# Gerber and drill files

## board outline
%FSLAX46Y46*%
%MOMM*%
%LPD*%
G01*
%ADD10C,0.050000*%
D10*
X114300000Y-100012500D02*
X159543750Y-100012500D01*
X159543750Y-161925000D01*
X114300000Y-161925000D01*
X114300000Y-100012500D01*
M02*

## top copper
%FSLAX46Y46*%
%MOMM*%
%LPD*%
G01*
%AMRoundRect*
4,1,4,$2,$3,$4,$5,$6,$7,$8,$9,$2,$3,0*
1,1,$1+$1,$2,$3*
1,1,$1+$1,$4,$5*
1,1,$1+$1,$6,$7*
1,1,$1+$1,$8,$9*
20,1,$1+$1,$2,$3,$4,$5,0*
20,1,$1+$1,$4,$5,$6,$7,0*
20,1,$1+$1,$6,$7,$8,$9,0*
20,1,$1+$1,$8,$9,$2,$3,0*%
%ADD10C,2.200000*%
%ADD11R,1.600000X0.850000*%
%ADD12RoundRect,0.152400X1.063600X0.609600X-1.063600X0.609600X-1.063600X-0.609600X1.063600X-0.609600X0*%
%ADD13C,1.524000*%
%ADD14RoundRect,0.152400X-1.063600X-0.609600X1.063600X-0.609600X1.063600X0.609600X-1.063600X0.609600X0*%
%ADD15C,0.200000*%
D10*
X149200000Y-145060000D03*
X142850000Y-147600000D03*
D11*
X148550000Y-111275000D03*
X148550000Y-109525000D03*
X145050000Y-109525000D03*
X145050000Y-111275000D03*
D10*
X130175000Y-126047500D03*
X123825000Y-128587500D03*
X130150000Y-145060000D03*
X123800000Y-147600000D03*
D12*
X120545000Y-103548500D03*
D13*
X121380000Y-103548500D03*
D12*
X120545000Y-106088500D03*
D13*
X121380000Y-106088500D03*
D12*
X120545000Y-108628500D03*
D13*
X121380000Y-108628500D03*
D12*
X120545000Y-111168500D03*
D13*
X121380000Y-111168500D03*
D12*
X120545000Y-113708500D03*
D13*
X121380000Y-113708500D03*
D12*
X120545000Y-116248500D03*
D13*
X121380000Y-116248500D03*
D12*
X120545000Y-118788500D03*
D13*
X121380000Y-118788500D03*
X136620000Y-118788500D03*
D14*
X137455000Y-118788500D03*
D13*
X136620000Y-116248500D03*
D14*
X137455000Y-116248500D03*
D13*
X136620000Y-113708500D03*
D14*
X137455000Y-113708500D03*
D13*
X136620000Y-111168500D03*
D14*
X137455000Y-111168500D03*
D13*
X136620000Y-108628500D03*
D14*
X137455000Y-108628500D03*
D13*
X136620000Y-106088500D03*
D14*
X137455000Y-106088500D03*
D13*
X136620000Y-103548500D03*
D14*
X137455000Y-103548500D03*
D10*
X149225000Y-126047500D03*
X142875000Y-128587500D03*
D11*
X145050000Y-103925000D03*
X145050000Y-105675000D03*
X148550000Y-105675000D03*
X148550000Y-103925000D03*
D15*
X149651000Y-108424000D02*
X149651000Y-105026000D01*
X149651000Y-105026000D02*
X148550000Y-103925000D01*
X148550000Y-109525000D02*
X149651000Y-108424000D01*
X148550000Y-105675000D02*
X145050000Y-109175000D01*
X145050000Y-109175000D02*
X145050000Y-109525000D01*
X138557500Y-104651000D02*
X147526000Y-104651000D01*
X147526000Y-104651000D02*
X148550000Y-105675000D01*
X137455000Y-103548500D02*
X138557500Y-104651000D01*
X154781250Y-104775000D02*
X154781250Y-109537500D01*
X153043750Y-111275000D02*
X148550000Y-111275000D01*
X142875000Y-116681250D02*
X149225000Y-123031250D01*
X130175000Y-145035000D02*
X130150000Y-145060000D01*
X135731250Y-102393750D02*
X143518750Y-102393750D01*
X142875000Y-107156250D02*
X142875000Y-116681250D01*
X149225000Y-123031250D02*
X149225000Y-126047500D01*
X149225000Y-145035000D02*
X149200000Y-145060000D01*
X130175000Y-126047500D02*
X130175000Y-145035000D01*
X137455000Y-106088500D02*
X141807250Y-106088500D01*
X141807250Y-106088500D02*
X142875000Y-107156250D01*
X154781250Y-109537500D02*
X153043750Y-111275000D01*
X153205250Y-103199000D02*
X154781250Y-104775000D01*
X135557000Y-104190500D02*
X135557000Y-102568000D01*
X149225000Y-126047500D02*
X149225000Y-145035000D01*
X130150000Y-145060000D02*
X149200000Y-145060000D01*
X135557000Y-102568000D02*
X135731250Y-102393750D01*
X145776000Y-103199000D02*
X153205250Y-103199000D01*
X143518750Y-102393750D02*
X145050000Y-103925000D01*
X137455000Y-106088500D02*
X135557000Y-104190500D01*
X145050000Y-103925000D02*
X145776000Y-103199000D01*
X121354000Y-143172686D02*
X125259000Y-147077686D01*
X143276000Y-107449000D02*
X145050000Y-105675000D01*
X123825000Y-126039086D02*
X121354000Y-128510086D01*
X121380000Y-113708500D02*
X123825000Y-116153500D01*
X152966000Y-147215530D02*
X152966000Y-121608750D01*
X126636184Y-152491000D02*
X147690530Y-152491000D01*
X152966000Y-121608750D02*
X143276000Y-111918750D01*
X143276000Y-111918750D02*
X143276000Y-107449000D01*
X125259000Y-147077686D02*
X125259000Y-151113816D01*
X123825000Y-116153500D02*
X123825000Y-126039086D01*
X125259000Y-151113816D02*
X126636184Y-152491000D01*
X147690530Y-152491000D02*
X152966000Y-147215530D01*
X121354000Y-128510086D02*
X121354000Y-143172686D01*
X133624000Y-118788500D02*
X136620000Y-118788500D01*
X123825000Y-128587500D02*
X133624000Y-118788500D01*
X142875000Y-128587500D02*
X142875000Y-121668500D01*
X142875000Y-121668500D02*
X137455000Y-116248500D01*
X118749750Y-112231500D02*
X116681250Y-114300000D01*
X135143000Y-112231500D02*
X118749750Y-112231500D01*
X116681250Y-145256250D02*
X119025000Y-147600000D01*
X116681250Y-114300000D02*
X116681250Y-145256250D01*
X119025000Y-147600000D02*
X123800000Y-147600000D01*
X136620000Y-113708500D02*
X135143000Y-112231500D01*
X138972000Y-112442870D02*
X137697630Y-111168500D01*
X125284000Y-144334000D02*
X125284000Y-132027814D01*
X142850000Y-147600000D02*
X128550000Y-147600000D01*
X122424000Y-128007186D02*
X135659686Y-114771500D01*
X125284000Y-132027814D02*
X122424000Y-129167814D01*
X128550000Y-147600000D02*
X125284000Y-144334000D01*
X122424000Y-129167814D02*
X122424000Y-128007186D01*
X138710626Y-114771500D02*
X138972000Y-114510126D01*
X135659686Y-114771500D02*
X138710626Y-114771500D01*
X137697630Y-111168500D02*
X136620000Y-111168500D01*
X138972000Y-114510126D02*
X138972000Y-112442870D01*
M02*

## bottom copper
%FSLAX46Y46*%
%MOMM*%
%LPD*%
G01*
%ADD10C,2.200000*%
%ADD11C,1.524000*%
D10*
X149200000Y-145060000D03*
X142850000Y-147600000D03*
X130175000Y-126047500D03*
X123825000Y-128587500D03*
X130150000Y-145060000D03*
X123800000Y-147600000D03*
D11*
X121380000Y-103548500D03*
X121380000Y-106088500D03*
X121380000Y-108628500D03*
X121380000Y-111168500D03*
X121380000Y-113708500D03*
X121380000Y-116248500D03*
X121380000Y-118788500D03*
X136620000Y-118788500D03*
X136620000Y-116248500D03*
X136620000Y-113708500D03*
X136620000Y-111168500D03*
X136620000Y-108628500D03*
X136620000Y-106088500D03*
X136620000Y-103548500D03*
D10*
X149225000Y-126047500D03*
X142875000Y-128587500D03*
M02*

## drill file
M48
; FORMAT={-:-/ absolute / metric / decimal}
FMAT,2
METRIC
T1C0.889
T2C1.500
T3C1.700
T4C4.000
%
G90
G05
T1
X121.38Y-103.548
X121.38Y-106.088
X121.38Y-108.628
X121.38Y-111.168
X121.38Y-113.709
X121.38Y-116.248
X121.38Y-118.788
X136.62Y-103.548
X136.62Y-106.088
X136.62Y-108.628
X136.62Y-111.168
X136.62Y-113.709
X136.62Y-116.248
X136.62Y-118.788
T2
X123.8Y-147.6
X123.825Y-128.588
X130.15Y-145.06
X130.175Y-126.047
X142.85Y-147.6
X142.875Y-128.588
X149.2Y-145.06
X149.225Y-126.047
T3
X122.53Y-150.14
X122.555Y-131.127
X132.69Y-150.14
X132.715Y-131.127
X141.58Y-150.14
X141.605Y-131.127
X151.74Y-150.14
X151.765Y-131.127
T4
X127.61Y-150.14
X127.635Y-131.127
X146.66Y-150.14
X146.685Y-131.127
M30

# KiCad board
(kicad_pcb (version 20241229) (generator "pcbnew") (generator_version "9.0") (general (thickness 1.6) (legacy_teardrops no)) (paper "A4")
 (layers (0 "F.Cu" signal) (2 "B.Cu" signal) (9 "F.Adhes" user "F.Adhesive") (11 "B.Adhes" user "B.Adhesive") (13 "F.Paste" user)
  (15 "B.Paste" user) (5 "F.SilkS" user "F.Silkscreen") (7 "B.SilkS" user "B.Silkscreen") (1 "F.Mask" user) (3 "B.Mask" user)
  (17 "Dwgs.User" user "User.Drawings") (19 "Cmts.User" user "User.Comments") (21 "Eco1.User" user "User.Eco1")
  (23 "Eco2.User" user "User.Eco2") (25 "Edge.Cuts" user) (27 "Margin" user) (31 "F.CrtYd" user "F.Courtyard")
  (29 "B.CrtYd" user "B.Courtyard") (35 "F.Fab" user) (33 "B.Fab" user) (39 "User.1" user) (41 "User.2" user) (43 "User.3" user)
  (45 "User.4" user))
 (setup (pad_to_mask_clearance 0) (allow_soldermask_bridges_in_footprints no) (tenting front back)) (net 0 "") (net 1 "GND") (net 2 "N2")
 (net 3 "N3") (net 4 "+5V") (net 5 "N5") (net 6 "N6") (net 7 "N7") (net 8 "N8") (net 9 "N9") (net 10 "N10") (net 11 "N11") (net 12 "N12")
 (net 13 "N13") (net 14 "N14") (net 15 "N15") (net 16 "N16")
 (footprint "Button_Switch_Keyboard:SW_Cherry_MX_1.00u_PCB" (layer "F.Cu") (at 149.2 145.06)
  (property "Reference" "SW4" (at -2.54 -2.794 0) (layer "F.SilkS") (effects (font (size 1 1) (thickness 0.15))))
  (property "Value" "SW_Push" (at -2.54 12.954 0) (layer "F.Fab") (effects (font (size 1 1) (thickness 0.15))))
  (pad "" np_thru_hole circle (at -7.62 5.08) (size 1.7 1.7) (drill 1.7) (layers "*.Cu" "*.Mask"))
  (pad "" np_thru_hole circle (at -2.54 5.08) (size 4 4) (drill 4) (layers "*.Cu" "*.Mask"))
  (pad "" np_thru_hole circle (at 2.54 5.08) (size 1.7 1.7) (drill 1.7) (layers "*.Cu" "*.Mask"))
  (pad "1" thru_hole circle (at 0 0) (size 2.2 2.2) (drill 1.5) (layers "*.Cu" "*.Mask") (remove_unused_layers no) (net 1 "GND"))
  (pad "2" thru_hole circle (at -6.35 2.54) (size 2.2 2.2) (drill 1.5) (layers "*.Cu" "*.Mask") (remove_unused_layers no) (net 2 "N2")))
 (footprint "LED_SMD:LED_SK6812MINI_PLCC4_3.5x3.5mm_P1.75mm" (layer "F.Cu") (at 146.8 110.4 180)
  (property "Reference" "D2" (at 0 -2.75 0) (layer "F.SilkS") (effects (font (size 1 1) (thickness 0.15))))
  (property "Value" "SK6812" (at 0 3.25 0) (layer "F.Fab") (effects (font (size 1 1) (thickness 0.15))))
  (pad "1" smd rect (at -1.75 -0.875 180) (size 1.6 0.85) (layers "F.Cu" "F.Mask" "F.Paste") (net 1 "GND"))
  (pad "2" smd rect (at -1.75 0.875 180) (size 1.6 0.85) (layers "F.Cu" "F.Mask" "F.Paste") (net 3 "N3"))
  (pad "3" smd rect (at 1.75 0.875 180) (size 1.6 0.85) (layers "F.Cu" "F.Mask" "F.Paste") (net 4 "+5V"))
  (pad "4" smd rect (at 1.75 -0.875 180) (size 1.6 0.85) (layers "F.Cu" "F.Mask" "F.Paste") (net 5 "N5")))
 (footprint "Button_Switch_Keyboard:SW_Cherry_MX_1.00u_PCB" (layer "F.Cu") (at 130.175 126.0475)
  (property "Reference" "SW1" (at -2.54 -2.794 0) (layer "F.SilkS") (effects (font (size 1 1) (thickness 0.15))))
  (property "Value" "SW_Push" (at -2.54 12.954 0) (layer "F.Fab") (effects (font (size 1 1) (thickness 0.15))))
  (pad "" np_thru_hole circle (at -7.62 5.08) (size 1.7 1.7) (drill 1.7) (layers "*.Cu" "*.Mask"))
  (pad "" np_thru_hole circle (at -2.54 5.08) (size 4 4) (drill 4) (layers "*.Cu" "*.Mask"))
  (pad "" np_thru_hole circle (at 2.54 5.08) (size 1.7 1.7) (drill 1.7) (layers "*.Cu" "*.Mask"))
  (pad "1" thru_hole circle (at 0 0) (size 2.2 2.2) (drill 1.5) (layers "*.Cu" "*.Mask") (remove_unused_layers no) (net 1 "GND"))
  (pad "2" thru_hole circle (at -6.35 2.54) (size 2.2 2.2) (drill 1.5) (layers "*.Cu" "*.Mask") (remove_unused_layers no) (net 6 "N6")))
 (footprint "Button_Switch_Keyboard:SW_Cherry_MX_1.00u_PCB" (layer "F.Cu") (at 130.15 145.06)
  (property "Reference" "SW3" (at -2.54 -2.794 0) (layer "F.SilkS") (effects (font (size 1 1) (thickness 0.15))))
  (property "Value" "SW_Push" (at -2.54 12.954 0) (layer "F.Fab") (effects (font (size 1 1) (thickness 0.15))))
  (pad "" np_thru_hole circle (at -7.62 5.08) (size 1.7 1.7) (drill 1.7) (layers "*.Cu" "*.Mask"))
  (pad "" np_thru_hole circle (at -2.54 5.08) (size 4 4) (drill 4) (layers "*.Cu" "*.Mask"))
  (pad "" np_thru_hole circle (at 2.54 5.08) (size 1.7 1.7) (drill 1.7) (layers "*.Cu" "*.Mask"))
  (pad "1" thru_hole circle (at 0 0) (size 2.2 2.2) (drill 1.5) (layers "*.Cu" "*.Mask") (remove_unused_layers no) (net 1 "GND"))
  (pad "2" thru_hole circle (at -6.35 2.54) (size 2.2 2.2) (drill 1.5) (layers "*.Cu" "*.Mask") (remove_unused_layers no) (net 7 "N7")))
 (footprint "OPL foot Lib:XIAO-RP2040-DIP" (layer "F.Cu") (at 129 111.1685)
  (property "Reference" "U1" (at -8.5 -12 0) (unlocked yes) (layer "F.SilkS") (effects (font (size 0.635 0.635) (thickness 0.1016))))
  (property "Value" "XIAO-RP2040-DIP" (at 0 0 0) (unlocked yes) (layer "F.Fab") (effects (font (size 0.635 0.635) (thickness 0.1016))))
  (pad "1" smd roundrect (at -8.455 -7.62 180) (size 2.432 1.524) (layers "F.Cu" "F.Mask") (roundrect_rratio 0.1) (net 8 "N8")
   (thermal_bridge_angle 45))
  (pad "1" thru_hole circle (at -7.62 -7.62 180) (size 1.524 1.524) (drill 0.889) (layers "*.Cu" "*.Mask") (remove_unused_layers no)
   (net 8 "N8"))
  (pad "2" smd roundrect (at -8.455 -5.08 180) (size 2.432 1.524) (layers "F.Cu" "F.Mask") (roundrect_rratio 0.1) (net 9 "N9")
   (thermal_bridge_angle 45))
  (pad "2" thru_hole circle (at -7.62 -5.08 180) (size 1.524 1.524) (drill 0.889) (layers "*.Cu" "*.Mask") (remove_unused_layers no)
   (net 9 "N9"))
  (pad "3" smd roundrect (at -8.455 -2.54 180) (size 2.432 1.524) (layers "F.Cu" "F.Mask") (roundrect_rratio 0.1) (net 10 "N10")
   (thermal_bridge_angle 45))
  (pad "3" thru_hole circle (at -7.62 -2.54 180) (size 1.524 1.524) (drill 0.889) (layers "*.Cu" "*.Mask") (remove_unused_layers no)
   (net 10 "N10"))
  (pad "4" smd roundrect (at -8.455 0 180) (size 2.432 1.524) (layers "F.Cu" "F.Mask") (roundrect_rratio 0.1) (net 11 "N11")
   (thermal_bridge_angle 45))
  (pad "4" thru_hole circle (at -7.62 0 180) (size 1.524 1.524) (drill 0.889) (layers "*.Cu" "*.Mask") (remove_unused_layers no)
   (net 11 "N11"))
  (pad "5" smd roundrect (at -8.455 2.54 180) (size 2.432 1.524) (layers "F.Cu" "F.Mask") (roundrect_rratio 0.1) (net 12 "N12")
   (thermal_bridge_angle 45))
  (pad "5" thru_hole circle (at -7.62 2.54 180) (size 1.524 1.524) (drill 0.889) (layers "*.Cu" "*.Mask") (remove_unused_layers no)
   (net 12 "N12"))
  (pad "6" smd roundrect (at -8.455 5.08 180) (size 2.432 1.524) (layers "F.Cu" "F.Mask") (roundrect_rratio 0.1) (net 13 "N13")
   (thermal_bridge_angle 45))
  (pad "6" thru_hole circle (at -7.62 5.08 180) (size 1.524 1.524) (drill 0.889) (layers "*.Cu" "*.Mask") (remove_unused_layers no)
   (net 13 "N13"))
  (pad "7" smd roundrect (at -8.455 7.62 180) (size 2.432 1.524) (layers "F.Cu" "F.Mask") (roundrect_rratio 0.1) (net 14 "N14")
   (thermal_bridge_angle 45))
  (pad "7" thru_hole circle (at -7.62 7.62 180) (size 1.524 1.524) (drill 0.889) (layers "*.Cu" "*.Mask") (remove_unused_layers no)
   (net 14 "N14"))
  (pad "8" thru_hole circle (at 7.62 7.62) (size 1.524 1.524) (drill 0.889) (layers "*.Cu" "*.Mask") (remove_unused_layers no) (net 6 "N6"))
  (pad "8" smd roundrect (at 8.455 7.62) (size 2.432 1.524) (layers "F.Cu" "F.Mask") (roundrect_rratio 0.1) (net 6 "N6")
   (thermal_bridge_angle 45))
  (pad "9" thru_hole circle (at 7.62 5.08) (size 1.524 1.524) (drill 0.889) (layers "*.Cu" "*.Mask") (remove_unused_layers no)
   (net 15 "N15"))
  (pad "9" smd roundrect (at 8.455 5.08) (size 2.432 1.524) (layers "F.Cu" "F.Mask") (roundrect_rratio 0.1) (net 15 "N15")
   (thermal_bridge_angle 45))
  (pad "10" thru_hole circle (at 7.62 2.54) (size 1.524 1.524) (drill 0.889) (layers "*.Cu" "*.Mask") (remove_unused_layers no) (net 7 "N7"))
  (pad "10" smd roundrect (at 8.455 2.54) (size 2.432 1.524) (layers "F.Cu" "F.Mask") (roundrect_rratio 0.1) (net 7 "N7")
   (thermal_bridge_angle 45))
  (pad "11" thru_hole circle (at 7.62 0) (size 1.524 1.524) (drill 0.889) (layers "*.Cu" "*.Mask") (remove_unused_layers no) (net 2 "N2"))
  (pad "11" smd roundrect (at 8.455 0) (size 2.432 1.524) (layers "F.Cu" "F.Mask") (roundrect_rratio 0.1) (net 2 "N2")
   (thermal_bridge_angle 45))
  (pad "12" thru_hole circle (at 7.62 -2.54) (size 1.524 1.524) (drill 0.889) (layers "*.Cu" "*.Mask") (remove_unused_layers no)
   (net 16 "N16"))
  (pad "12" smd roundrect (at 8.455 -2.54) (size 2.432 1.524) (layers "F.Cu" "F.Mask") (roundrect_rratio 0.1) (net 16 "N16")
   (thermal_bridge_angle 45))
  (pad "13" thru_hole circle (at 7.62 -5.08) (size 1.524 1.524) (drill 0.889) (layers "*.Cu" "*.Mask") (remove_unused_layers no)
   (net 1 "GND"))
  (pad "13" smd roundrect (at 8.455 -5.08) (size 2.432 1.524) (layers "F.Cu" "F.Mask") (roundrect_rratio 0.1) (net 1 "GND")
   (thermal_bridge_angle 45))
  (pad "14" thru_hole circle (at 7.62 -7.62) (size 1.524 1.524) (drill 0.889) (layers "*.Cu" "*.Mask") (remove_unused_layers no)
   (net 4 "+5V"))
  (pad "14" smd roundrect (at 8.455 -7.62) (size 2.432 1.524) (layers "F.Cu" "F.Mask") (roundrect_rratio 0.1) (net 4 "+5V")
   (thermal_bridge_angle 45)))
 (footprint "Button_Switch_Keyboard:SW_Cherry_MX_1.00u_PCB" (layer "F.Cu") (at 149.225 126.0475)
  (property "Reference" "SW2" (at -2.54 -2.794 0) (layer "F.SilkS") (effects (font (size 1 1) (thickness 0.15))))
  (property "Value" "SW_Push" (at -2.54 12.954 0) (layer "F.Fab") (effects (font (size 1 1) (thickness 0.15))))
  (pad "" np_thru_hole circle (at -7.62 5.08) (size 1.7 1.7) (drill 1.7) (layers "*.Cu" "*.Mask"))
  (pad "" np_thru_hole circle (at -2.54 5.08) (size 4 4) (drill 4) (layers "*.Cu" "*.Mask"))
  (pad "" np_thru_hole circle (at 2.54 5.08) (size 1.7 1.7) (drill 1.7) (layers "*.Cu" "*.Mask"))
  (pad "1" thru_hole circle (at 0 0) (size 2.2 2.2) (drill 1.5) (layers "*.Cu" "*.Mask") (remove_unused_layers no) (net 1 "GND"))
  (pad "2" thru_hole circle (at -6.35 2.54) (size 2.2 2.2) (drill 1.5) (layers "*.Cu" "*.Mask") (remove_unused_layers no) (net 15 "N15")))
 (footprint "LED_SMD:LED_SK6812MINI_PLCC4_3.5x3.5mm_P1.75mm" (layer "F.Cu") (at 146.8 104.8)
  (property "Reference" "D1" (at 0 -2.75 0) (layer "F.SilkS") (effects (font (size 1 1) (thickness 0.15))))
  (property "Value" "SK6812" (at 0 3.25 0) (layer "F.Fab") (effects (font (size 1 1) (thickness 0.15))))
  (pad "1" smd rect (at -1.75 -0.875) (size 1.6 0.85) (layers "F.Cu" "F.Mask" "F.Paste") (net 1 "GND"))
  (pad "2" smd rect (at -1.75 0.875) (size 1.6 0.85) (layers "F.Cu" "F.Mask" "F.Paste") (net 12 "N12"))
  (pad "3" smd rect (at 1.75 0.875) (size 1.6 0.85) (layers "F.Cu" "F.Mask" "F.Paste") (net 4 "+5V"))
  (pad "4" smd rect (at 1.75 -0.875) (size 1.6 0.85) (layers "F.Cu" "F.Mask" "F.Paste") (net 3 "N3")))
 (gr_rect (start 114.3 100.0125) (end 159.54375 161.925) (stroke (width 0.05) (type default)) (fill no) (layer "Edge.Cuts"))
 (segment (start 149.651 108.424) (end 149.651 105.026) (width 0.2) (layer "F.Cu") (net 3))
 (segment (start 149.651 105.026) (end 148.55 103.925) (width 0.2) (layer "F.Cu") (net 3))
 (segment (start 148.55 109.525) (end 149.651 108.424) (width 0.2) (layer "F.Cu") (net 3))
 (segment (start 148.55 105.675) (end 145.05 109.175) (width 0.2) (layer "F.Cu") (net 4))
 (segment (start 145.05 109.175) (end 145.05 109.525) (width 0.2) (layer "F.Cu") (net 4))
 (segment (start 138.5575 104.651) (end 147.526 104.651) (width 0.2) (layer "F.Cu") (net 4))
 (segment (start 147.526 104.651) (end 148.55 105.675) (width 0.2) (layer "F.Cu") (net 4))
 (segment (start 137.455 103.5485) (end 138.5575 104.651) (width 0.2) (layer "F.Cu") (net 4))
 (segment (start 154.78125 104.775) (end 154.78125 109.5375) (width 0.2) (layer "F.Cu") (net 1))
 (segment (start 153.04375 111.275) (end 148.55 111.275) (width 0.2) (layer "F.Cu") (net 1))
 (segment (start 142.875 116.68125) (end 149.225 123.03125) (width 0.2) (layer "F.Cu") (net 1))
 (segment (start 130.175 145.035) (end 130.15 145.06) (width 0.2) (layer "F.Cu") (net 1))
 (segment (start 135.73125 102.39375) (end 143.51875 102.39375) (width 0.2) (layer "F.Cu") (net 1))
 (segment (start 142.875 107.15625) (end 142.875 116.68125) (width 0.2) (layer "F.Cu") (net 1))
 (segment (start 149.225 123.03125) (end 149.225 126.0475) (width 0.2) (layer "F.Cu") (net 1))
 (segment (start 149.225 145.035) (end 149.2 145.06) (width 0.2) (layer "F.Cu") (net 1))
 (segment (start 130.175 126.0475) (end 130.175 145.035) (width 0.2) (layer "F.Cu") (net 1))
 (segment (start 137.455 106.0885) (end 141.80725 106.0885) (width 0.2) (layer "F.Cu") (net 1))
 (segment (start 141.80725 106.0885) (end 142.875 107.15625) (width 0.2) (layer "F.Cu") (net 1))
 (segment (start 154.78125 109.5375) (end 153.04375 111.275) (width 0.2) (layer "F.Cu") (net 1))
 (segment (start 153.20525 103.199) (end 154.78125 104.775) (width 0.2) (layer "F.Cu") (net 1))
 (segment (start 135.557 104.1905) (end 135.557 102.568) (width 0.2) (layer "F.Cu") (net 1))
 (segment (start 149.225 126.0475) (end 149.225 145.035) (width 0.2) (layer "F.Cu") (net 1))
 (segment (start 130.15 145.06) (end 149.2 145.06) (width 0.2) (layer "F.Cu") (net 1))
 (segment (start 135.557 102.568) (end 135.73125 102.39375) (width 0.2) (layer "F.Cu") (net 1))
 (segment (start 145.776 103.199) (end 153.20525 103.199) (width 0.2) (layer "F.Cu") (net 1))
 (segment (start 143.51875 102.39375) (end 145.05 103.925) (width 0.2) (layer "F.Cu") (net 1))
 (segment (start 137.455 106.0885) (end 135.557 104.1905) (width 0.2) (layer "F.Cu") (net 1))
 (segment (start 145.05 103.925) (end 145.776 103.199) (width 0.2) (layer "F.Cu") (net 1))
 (segment (start 121.354 143.172686) (end 125.259 147.077686) (width 0.2) (layer "F.Cu") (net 12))
 (segment (start 143.276 107.449) (end 145.05 105.675) (width 0.2) (layer "F.Cu") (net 12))
 (segment (start 123.825 126.039086) (end 121.354 128.510086) (width 0.2) (layer "F.Cu") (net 12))
 (segment (start 121.38 113.7085) (end 123.825 116.1535) (width 0.2) (layer "F.Cu") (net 12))
 (segment (start 152.966 147.21553) (end 152.966 121.60875) (width 0.2) (layer "F.Cu") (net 12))
 (segment (start 126.636184 152.491) (end 147.69053 152.491) (width 0.2) (layer "F.Cu") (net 12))
 (segment (start 152.966 121.60875) (end 143.276 111.91875) (width 0.2) (layer "F.Cu") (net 12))
 (segment (start 143.276 111.91875) (end 143.276 107.449) (width 0.2) (layer "F.Cu") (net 12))
 (segment (start 125.259 147.077686) (end 125.259 151.113816) (width 0.2) (layer "F.Cu") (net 12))
 (segment (start 123.825 116.1535) (end 123.825 126.039086) (width 0.2) (layer "F.Cu") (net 12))
 (segment (start 125.259 151.113816) (end 126.636184 152.491) (width 0.2) (layer "F.Cu") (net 12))
 (segment (start 147.69053 152.491) (end 152.966 147.21553) (width 0.2) (layer "F.Cu") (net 12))
 (segment (start 121.354 128.510086) (end 121.354 143.172686) (width 0.2) (layer "F.Cu") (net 12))
 (segment (start 133.624 118.7885) (end 136.62 118.7885) (width 0.2) (layer "F.Cu") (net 6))
 (segment (start 123.825 128.5875) (end 133.624 118.7885) (width 0.2) (layer "F.Cu") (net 6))
 (segment (start 142.875 128.5875) (end 142.875 121.6685) (width 0.2) (layer "F.Cu") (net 15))
 (segment (start 142.875 121.6685) (end 137.455 116.2485) (width 0.2) (layer "F.Cu") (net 15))
 (segment (start 118.74975 112.2315) (end 116.68125 114.3) (width 0.2) (layer "F.Cu") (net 7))
 (segment (start 135.143 112.2315) (end 118.74975 112.2315) (width 0.2) (layer "F.Cu") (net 7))
 (segment (start 116.68125 145.25625) (end 119.025 147.6) (width 0.2) (layer "F.Cu") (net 7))
 (segment (start 116.68125 114.3) (end 116.68125 145.25625) (width 0.2) (layer "F.Cu") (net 7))
 (segment (start 119.025 147.6) (end 123.8 147.6) (width 0.2) (layer "F.Cu") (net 7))
 (segment (start 136.62 113.7085) (end 135.143 112.2315) (width 0.2) (layer "F.Cu") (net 7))
 (segment (start 138.972 112.44287) (end 137.69763 111.1685) (width 0.2) (layer "F.Cu") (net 2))
 (segment (start 125.284 144.334) (end 125.284 132.027814) (width 0.2) (layer "F.Cu") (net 2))
 (segment (start 142.85 147.6) (end 128.55 147.6) (width 0.2) (layer "F.Cu") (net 2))
 (segment (start 122.424 128.007186) (end 135.659686 114.7715) (width 0.2) (layer "F.Cu") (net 2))
 (segment (start 125.284 132.027814) (end 122.424 129.167814) (width 0.2) (layer "F.Cu") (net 2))
 (segment (start 128.55 147.6) (end 125.284 144.334) (width 0.2) (layer "F.Cu") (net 2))
 (segment (start 122.424 129.167814) (end 122.424 128.007186) (width 0.2) (layer "F.Cu") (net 2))
 (segment (start 138.710626 114.7715) (end 138.972 114.510126) (width 0.2) (layer "F.Cu") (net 2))
 (segment (start 135.659686 114.7715) (end 138.710626 114.7715) (width 0.2) (layer "F.Cu") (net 2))
 (segment (start 137.69763 111.1685) (end 136.62 111.1685) (width 0.2) (layer "F.Cu") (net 2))
 (segment (start 138.972 114.510126) (end 138.972 112.44287) (width 0.2) (layer "F.Cu") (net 2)))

